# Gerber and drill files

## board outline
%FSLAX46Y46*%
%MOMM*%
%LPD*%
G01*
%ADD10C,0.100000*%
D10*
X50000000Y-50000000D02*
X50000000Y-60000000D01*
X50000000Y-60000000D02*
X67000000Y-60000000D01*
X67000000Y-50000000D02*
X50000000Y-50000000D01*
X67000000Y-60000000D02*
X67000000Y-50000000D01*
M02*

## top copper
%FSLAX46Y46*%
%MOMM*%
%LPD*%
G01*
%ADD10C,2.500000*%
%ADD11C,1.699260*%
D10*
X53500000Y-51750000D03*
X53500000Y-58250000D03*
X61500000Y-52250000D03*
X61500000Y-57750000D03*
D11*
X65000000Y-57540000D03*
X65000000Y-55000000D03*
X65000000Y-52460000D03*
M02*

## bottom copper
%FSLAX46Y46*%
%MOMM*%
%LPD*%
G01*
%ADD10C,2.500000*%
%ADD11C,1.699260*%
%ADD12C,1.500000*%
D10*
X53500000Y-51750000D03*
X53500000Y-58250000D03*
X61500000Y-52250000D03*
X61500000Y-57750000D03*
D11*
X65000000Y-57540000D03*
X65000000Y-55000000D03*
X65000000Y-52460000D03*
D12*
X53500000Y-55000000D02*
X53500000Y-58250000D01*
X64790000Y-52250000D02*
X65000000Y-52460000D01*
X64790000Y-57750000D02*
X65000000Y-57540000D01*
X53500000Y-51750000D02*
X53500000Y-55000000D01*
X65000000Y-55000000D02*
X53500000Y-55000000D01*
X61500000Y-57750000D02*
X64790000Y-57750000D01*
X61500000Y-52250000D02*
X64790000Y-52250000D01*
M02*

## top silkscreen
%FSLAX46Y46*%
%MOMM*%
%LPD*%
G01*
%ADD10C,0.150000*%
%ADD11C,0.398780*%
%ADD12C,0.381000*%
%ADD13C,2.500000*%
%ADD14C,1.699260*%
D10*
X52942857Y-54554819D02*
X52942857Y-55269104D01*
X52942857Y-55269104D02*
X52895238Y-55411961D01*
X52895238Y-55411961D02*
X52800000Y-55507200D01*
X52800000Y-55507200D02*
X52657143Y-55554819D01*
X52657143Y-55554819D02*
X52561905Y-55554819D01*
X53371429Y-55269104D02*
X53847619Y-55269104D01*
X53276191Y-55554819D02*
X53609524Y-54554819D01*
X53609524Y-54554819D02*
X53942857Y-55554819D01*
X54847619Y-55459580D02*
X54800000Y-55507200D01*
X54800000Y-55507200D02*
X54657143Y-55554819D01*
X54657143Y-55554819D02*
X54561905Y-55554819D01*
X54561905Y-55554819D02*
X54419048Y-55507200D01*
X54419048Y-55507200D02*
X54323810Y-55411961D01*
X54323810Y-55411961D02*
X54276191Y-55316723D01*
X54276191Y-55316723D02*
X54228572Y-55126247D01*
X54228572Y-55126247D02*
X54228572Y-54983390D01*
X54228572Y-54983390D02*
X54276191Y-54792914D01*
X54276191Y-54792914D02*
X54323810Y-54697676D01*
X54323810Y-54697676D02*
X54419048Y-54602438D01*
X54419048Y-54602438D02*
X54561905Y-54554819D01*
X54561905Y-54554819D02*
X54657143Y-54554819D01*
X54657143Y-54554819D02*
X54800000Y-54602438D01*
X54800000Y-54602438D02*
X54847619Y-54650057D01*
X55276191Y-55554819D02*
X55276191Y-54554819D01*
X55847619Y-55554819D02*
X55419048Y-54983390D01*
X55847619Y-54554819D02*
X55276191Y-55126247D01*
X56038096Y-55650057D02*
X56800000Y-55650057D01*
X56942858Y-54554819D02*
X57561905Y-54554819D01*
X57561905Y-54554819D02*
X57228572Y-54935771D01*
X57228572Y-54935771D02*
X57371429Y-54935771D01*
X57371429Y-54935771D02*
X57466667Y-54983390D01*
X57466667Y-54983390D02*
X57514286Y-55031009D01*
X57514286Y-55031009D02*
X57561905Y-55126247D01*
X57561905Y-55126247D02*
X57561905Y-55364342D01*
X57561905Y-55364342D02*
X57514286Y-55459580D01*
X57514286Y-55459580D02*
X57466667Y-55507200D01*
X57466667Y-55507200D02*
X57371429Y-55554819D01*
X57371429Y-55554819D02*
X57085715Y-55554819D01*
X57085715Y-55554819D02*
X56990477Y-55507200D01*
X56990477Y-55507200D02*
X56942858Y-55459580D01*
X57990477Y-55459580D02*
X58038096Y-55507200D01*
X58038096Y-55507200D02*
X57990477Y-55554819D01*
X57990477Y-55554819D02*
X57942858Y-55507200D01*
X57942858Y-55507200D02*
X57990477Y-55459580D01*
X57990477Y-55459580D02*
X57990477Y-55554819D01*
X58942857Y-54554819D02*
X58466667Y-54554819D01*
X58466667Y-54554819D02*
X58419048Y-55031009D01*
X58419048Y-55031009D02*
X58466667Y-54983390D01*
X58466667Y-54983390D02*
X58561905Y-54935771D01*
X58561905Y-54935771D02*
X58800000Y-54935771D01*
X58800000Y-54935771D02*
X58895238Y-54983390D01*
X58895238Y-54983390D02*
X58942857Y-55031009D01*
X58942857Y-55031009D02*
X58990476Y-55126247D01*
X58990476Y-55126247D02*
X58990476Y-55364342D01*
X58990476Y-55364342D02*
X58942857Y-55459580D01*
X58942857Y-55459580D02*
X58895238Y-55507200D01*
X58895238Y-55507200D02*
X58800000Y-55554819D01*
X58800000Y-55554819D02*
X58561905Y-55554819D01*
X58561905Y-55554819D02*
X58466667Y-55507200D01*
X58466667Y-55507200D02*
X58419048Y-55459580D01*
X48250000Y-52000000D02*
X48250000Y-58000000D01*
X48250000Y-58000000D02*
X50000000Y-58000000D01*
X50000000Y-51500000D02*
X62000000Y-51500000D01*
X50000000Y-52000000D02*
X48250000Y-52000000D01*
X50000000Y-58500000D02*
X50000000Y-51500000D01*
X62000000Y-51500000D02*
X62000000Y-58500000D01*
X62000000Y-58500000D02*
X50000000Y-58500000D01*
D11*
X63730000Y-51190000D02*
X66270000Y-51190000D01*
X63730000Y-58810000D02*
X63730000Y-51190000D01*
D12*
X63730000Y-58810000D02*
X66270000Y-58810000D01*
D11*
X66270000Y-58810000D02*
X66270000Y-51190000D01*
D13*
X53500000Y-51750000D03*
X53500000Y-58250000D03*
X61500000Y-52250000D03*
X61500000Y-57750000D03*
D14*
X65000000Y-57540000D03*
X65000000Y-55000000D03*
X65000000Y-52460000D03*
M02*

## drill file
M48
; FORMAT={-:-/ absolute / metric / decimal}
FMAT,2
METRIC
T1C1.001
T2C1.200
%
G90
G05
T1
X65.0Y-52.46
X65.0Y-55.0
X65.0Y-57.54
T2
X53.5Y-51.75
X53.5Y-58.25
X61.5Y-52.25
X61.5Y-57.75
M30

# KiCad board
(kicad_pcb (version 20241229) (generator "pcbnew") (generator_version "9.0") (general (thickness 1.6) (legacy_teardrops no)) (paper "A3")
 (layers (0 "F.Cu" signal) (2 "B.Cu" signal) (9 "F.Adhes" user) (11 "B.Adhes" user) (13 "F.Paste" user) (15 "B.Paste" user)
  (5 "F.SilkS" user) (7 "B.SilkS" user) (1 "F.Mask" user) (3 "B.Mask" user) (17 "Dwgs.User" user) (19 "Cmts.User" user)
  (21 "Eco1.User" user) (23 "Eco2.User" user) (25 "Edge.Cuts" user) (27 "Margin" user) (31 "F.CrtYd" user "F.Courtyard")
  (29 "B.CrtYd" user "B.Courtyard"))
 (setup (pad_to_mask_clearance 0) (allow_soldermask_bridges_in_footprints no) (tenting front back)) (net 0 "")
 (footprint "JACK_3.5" (layer "F.Cu") (at 56 55)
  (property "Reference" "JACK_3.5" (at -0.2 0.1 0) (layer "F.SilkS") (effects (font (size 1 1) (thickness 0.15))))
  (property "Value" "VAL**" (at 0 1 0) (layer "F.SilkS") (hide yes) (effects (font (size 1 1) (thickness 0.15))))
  (fp_line (start -7.75 -3) (end -7.75 3) (stroke (width 0.15) (type solid)) (layer "F.SilkS"))
  (fp_line (start -7.75 3) (end -6 3) (stroke (width 0.15) (type solid)) (layer "F.SilkS"))
  (fp_line (start -6 -3.5) (end 6 -3.5) (stroke (width 0.15) (type solid)) (layer "F.SilkS"))
  (fp_line (start -6 -3) (end -7.75 -3) (stroke (width 0.15) (type solid)) (layer "F.SilkS"))
  (fp_line (start -6 3.5) (end -6 -3.5) (stroke (width 0.15) (type solid)) (layer "F.SilkS"))
  (fp_line (start 6 -3.5) (end 6 3.5) (stroke (width 0.15) (type solid)) (layer "F.SilkS"))
  (fp_line (start 6 3.5) (end -6 3.5) (stroke (width 0.15) (type solid)) (layer "F.SilkS"))
  (pad "1" thru_hole circle (at -2.5 -3.25) (size 2.5 2.5) (drill 1.2) (layers "*.Cu" "*.Mask" "F.SilkS") (remove_unused_layers no))
  (pad "1" thru_hole circle (at -2.5 3.25) (size 2.5 2.5) (drill 1.2) (layers "*.Cu" "*.Mask" "F.SilkS") (remove_unused_layers no))
  (pad "2" thru_hole circle (at 5.5 -2.75) (size 2.5 2.5) (drill 1.2) (layers "*.Cu" "*.Mask" "F.SilkS") (remove_unused_layers no))
  (pad "3" thru_hole circle (at 5.5 2.75) (size 2.5 2.5) (drill 1.2) (layers "*.Cu" "*.Mask" "F.SilkS") (remove_unused_layers no)))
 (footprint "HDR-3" (layer "F.Cu") (at 65 55 90)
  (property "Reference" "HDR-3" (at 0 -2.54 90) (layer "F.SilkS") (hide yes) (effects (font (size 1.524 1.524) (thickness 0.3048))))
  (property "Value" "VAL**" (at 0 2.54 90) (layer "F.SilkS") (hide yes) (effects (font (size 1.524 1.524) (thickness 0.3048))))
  (fp_line (start 3.81 -1.27) (end 3.81 1.27) (stroke (width 0.39878) (type solid)) (layer "F.SilkS"))
  (fp_line (start -3.81 -1.27) (end 3.81 -1.27) (stroke (width 0.39878) (type solid)) (layer "F.SilkS"))
  (fp_line (start -3.81 -1.27) (end -3.81 1.27) (stroke (width 0.381) (type solid)) (layer "F.SilkS"))
  (fp_line (start -3.81 1.27) (end 3.81 1.27) (stroke (width 0.39878) (type solid)) (layer "F.SilkS"))
  (pad "1" thru_hole circle (at -2.54 0 90) (size 1.69926 1.69926) (drill 1.00076) (layers "*.Cu" "*.Mask" "F.SilkS")
   (remove_unused_layers no))
  (pad "2" thru_hole circle (at 0 0 90) (size 1.69926 1.69926) (drill 1.00076) (layers "*.Cu" "*.Mask" "F.SilkS") (remove_unused_layers no))
  (pad "3" thru_hole circle (at 2.54 0 90) (size 1.69926 1.69926) (drill 1.00076) (layers "*.Cu" "*.Mask" "F.SilkS")
   (remove_unused_layers no)))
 (gr_line (start 50 50) (end 50 60) (stroke (width 0.1) (type solid)) (layer "Edge.Cuts"))
 (gr_line (start 50 60) (end 67 60) (stroke (width 0.1) (type solid)) (layer "Edge.Cuts"))
 (gr_line (start 67 50) (end 50 50) (stroke (width 0.1) (type solid)) (layer "Edge.Cuts"))
 (gr_line (start 67 60) (end 67 50) (stroke (width 0.1) (type solid)) (layer "Edge.Cuts"))
 (segment (start 53.5 55) (end 53.5 58.25) (width 1.5) (layer "B.Cu") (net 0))
 (segment (start 64.79 52.25) (end 65 52.46) (width 1.5) (layer "B.Cu") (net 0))
 (segment (start 64.79 57.75) (end 65 57.54) (width 1.5) (layer "B.Cu") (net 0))
 (segment (start 53.5 51.75) (end 53.5 55) (width 1.5) (layer "B.Cu") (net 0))
 (segment (start 65 55) (end 53.5 55) (width 1.5) (layer "B.Cu") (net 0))
 (segment (start 61.5 57.75) (end 64.79 57.75) (width 1.5) (layer "B.Cu") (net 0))
 (segment (start 61.5 52.25) (end 64.79 52.25) (width 1.5) (layer "B.Cu") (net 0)))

